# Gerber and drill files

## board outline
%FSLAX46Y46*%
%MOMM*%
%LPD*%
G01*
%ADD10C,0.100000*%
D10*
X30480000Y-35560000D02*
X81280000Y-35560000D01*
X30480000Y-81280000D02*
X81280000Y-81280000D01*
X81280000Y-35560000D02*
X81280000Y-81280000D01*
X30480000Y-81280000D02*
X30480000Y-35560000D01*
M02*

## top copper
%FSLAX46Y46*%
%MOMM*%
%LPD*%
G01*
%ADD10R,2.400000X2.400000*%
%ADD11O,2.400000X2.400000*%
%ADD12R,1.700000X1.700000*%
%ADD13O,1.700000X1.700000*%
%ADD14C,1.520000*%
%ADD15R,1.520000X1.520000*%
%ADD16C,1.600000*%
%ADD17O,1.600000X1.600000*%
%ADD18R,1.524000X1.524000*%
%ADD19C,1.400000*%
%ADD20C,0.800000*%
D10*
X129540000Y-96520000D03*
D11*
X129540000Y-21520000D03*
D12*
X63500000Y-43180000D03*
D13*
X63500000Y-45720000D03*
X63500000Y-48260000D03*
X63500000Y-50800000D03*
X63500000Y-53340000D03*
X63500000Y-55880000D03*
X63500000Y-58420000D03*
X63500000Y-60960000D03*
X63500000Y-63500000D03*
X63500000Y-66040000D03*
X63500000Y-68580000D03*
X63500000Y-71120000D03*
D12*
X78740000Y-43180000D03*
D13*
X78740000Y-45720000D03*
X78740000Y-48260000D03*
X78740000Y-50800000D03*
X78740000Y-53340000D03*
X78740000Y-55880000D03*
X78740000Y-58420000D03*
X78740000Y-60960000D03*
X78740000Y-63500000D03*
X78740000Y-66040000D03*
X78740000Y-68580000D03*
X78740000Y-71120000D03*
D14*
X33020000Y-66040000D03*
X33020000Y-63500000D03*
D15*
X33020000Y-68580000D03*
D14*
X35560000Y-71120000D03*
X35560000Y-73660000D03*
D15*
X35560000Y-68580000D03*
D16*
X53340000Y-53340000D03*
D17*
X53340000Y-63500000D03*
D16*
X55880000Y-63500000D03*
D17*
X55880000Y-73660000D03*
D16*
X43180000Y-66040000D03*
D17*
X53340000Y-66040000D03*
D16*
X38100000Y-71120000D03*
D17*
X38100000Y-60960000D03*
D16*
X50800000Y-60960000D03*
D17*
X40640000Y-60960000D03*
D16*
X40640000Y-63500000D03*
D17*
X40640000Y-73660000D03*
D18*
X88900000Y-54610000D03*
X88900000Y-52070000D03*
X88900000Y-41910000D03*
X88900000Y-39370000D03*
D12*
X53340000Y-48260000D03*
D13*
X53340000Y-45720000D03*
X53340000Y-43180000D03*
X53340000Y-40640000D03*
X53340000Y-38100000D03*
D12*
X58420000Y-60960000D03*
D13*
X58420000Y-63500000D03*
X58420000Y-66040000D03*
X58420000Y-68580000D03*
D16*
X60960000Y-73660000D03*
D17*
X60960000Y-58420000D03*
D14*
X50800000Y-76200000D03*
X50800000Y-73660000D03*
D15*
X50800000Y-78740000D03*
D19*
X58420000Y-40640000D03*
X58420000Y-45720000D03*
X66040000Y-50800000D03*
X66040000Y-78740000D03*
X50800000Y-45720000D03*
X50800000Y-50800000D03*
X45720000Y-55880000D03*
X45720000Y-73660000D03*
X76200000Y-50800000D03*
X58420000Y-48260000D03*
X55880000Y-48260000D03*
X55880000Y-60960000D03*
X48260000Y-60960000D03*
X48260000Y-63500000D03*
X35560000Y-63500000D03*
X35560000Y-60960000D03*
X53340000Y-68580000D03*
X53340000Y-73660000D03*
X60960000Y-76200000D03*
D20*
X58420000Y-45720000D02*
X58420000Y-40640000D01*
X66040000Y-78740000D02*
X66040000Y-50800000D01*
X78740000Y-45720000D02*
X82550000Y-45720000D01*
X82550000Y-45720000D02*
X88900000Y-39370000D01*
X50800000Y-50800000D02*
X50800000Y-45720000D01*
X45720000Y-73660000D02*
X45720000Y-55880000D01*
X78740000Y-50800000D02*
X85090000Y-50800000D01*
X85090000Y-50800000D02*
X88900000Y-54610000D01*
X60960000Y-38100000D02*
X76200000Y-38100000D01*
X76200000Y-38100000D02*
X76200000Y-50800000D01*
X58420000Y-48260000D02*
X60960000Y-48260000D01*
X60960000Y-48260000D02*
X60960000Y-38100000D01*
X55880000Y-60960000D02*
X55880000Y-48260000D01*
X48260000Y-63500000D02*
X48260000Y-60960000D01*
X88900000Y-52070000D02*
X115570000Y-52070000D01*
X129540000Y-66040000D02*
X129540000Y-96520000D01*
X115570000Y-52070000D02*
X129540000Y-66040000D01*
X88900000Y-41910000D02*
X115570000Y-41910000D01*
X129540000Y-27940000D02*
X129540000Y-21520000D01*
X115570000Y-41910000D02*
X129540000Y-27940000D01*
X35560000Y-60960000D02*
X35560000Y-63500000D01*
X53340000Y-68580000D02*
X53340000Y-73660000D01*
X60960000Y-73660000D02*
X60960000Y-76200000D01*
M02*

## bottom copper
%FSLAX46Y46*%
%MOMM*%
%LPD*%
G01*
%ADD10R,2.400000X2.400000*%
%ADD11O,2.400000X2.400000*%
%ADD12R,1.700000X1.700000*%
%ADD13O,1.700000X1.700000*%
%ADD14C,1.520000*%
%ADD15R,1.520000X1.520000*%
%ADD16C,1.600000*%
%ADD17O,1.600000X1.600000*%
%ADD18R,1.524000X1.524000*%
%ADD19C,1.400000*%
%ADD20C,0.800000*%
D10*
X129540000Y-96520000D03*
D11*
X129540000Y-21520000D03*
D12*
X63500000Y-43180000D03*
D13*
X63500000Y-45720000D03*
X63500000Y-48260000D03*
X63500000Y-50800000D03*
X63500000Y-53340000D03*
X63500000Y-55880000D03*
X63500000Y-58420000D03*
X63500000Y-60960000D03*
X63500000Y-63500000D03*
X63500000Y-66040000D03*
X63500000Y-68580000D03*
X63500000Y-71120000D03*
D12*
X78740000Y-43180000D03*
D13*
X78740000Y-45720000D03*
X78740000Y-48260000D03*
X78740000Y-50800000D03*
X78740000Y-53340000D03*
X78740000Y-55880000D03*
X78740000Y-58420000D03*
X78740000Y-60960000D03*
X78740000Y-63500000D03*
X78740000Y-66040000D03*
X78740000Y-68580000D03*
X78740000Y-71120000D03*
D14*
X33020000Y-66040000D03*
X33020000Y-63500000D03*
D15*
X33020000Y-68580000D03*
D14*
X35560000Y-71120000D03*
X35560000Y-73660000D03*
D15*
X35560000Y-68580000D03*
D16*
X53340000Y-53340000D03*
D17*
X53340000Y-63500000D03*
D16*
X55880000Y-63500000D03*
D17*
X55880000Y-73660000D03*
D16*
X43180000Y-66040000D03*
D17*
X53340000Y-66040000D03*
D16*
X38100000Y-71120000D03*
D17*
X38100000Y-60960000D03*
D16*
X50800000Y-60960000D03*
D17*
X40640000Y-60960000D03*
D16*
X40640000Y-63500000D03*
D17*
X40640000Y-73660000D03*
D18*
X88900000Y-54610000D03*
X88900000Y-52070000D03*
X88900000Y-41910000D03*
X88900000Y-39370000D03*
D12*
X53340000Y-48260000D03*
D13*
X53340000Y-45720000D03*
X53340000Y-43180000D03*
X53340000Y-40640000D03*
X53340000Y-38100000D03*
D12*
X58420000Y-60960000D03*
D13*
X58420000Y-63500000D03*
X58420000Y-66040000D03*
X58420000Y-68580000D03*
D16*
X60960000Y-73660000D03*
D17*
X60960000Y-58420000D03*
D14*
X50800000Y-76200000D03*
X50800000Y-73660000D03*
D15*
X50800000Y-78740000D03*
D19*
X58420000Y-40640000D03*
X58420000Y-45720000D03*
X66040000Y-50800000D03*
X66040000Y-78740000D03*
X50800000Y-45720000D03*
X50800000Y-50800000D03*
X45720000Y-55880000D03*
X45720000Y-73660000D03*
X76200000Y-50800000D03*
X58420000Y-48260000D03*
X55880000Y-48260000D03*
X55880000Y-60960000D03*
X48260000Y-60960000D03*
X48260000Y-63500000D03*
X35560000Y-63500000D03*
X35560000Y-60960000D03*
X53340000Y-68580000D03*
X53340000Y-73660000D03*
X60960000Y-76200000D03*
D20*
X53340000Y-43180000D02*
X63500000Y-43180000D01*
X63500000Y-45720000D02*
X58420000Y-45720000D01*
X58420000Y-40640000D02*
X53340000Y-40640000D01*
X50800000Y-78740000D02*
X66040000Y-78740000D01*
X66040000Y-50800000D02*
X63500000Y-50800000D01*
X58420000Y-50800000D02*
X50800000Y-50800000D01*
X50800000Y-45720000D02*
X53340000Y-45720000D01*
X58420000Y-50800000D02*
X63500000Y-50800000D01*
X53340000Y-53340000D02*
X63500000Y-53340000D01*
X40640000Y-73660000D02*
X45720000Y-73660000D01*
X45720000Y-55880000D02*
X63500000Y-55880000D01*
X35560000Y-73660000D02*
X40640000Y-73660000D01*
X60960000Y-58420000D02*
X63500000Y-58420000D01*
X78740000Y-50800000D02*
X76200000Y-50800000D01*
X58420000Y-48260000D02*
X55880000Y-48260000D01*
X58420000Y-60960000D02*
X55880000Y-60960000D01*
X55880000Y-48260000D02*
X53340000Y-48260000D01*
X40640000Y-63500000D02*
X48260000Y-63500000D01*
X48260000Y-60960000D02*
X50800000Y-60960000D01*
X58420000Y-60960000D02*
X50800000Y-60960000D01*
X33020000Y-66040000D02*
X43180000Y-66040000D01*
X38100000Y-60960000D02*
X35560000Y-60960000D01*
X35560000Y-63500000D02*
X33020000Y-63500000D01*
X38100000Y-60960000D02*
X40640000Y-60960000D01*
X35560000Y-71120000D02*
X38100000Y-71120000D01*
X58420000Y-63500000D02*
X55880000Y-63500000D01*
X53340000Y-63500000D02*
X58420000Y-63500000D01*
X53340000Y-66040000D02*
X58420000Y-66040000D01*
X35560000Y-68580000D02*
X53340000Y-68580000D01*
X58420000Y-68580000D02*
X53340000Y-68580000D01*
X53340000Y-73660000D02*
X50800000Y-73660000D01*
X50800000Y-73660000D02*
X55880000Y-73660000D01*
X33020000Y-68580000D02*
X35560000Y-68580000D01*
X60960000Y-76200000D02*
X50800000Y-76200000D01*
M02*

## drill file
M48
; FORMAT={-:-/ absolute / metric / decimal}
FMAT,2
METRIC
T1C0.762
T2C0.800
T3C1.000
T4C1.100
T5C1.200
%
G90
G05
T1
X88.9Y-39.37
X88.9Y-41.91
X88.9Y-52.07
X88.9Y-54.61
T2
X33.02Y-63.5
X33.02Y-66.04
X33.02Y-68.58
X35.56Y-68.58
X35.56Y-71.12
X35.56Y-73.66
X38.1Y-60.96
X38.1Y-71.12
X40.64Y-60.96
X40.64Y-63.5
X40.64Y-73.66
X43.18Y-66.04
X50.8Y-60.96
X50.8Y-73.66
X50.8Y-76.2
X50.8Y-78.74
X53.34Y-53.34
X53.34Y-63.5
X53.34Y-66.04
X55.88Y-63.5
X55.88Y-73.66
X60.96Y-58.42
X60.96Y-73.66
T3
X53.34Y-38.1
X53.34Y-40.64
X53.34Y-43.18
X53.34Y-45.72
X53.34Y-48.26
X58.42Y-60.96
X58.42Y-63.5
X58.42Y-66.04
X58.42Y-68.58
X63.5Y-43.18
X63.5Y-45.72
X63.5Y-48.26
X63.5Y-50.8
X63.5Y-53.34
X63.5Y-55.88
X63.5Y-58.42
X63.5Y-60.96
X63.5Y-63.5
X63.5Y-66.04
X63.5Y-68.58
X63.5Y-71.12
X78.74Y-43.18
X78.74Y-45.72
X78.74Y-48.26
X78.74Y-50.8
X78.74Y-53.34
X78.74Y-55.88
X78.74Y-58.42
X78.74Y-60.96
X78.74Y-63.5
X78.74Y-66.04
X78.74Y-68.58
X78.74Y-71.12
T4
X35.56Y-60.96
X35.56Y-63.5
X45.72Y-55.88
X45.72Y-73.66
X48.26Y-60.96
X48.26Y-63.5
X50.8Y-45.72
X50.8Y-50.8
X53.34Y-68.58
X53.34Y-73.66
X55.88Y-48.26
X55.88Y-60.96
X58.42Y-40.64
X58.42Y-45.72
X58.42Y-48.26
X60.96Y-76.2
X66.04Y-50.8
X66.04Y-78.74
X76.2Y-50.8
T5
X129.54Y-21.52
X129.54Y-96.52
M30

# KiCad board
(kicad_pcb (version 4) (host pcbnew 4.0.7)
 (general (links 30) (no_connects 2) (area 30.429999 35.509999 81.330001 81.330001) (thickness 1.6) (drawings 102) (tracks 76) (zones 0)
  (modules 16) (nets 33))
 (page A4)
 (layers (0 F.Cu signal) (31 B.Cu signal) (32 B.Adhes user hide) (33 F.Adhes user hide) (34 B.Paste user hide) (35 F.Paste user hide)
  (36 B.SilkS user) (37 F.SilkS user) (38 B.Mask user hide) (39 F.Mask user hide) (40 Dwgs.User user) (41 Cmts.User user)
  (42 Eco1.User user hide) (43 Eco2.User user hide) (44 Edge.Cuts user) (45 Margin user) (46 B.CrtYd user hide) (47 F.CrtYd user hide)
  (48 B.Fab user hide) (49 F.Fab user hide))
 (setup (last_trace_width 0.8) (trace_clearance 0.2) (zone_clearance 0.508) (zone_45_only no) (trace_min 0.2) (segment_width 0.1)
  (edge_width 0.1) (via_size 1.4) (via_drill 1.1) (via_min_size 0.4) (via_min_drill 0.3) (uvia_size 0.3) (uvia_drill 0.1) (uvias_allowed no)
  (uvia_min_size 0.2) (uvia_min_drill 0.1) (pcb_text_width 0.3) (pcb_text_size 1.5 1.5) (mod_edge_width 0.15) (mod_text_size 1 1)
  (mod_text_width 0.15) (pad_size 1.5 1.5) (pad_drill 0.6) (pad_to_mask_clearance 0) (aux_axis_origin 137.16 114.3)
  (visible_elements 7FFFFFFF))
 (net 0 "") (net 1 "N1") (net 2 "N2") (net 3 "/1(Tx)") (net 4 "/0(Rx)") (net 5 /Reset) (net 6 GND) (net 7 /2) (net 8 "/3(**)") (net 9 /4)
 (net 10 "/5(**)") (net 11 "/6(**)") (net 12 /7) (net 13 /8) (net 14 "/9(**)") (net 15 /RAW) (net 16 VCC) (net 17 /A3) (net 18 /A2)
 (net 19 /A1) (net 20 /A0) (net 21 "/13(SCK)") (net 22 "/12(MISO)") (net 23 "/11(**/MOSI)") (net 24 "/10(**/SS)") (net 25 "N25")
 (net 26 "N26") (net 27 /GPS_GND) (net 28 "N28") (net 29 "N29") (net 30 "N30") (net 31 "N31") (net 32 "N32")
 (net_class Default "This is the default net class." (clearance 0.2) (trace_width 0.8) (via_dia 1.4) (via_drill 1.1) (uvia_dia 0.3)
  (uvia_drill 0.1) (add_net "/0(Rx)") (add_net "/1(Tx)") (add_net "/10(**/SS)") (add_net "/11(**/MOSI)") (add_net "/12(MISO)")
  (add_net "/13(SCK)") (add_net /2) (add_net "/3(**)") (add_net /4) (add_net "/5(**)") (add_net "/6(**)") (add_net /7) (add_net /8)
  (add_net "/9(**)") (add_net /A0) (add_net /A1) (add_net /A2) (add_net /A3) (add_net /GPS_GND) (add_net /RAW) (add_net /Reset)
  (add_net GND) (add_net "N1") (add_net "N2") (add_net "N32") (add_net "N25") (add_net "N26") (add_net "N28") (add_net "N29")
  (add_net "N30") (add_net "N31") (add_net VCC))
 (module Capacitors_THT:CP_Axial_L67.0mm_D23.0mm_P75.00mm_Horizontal (layer F.Cu) (at 129.54 96.52 90)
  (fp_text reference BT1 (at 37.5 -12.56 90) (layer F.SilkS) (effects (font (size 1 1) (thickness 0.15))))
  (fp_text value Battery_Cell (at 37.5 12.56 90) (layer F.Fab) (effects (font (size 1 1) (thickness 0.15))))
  (pad 1 thru_hole rect (at 0 0 90) (size 2.4 2.4) (drill 1.2) (layers *.Cu *.Mask) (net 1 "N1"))
  (pad 2 thru_hole oval (at 75 0 90) (size 2.4 2.4) (drill 1.2) (layers *.Cu *.Mask) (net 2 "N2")))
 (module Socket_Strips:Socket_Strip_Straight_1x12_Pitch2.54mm (layer F.Cu) (at 63.5 43.18)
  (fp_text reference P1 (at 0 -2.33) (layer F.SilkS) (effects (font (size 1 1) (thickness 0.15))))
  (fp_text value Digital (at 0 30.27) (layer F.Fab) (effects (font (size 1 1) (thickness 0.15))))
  (pad 1 thru_hole rect (at 0 0) (size 1.7 1.7) (drill 1) (layers *.Cu *.Mask) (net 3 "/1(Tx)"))
  (pad 2 thru_hole oval (at 0 2.54) (size 1.7 1.7) (drill 1) (layers *.Cu *.Mask) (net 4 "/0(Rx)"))
  (pad 3 thru_hole oval (at 0 5.08) (size 1.7 1.7) (drill 1) (layers *.Cu *.Mask) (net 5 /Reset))
  (pad 4 thru_hole oval (at 0 7.62) (size 1.7 1.7) (drill 1) (layers *.Cu *.Mask) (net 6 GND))
  (pad 5 thru_hole oval (at 0 10.16) (size 1.7 1.7) (drill 1) (layers *.Cu *.Mask) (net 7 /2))
  (pad 6 thru_hole oval (at 0 12.7) (size 1.7 1.7) (drill 1) (layers *.Cu *.Mask) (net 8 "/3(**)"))
  (pad 7 thru_hole oval (at 0 15.24) (size 1.7 1.7) (drill 1) (layers *.Cu *.Mask) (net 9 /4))
  (pad 8 thru_hole oval (at 0 17.78) (size 1.7 1.7) (drill 1) (layers *.Cu *.Mask) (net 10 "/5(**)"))
  (pad 9 thru_hole oval (at 0 20.32) (size 1.7 1.7) (drill 1) (layers *.Cu *.Mask) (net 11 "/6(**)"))
  (pad 10 thru_hole oval (at 0 22.86) (size 1.7 1.7) (drill 1) (layers *.Cu *.Mask) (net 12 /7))
  (pad 11 thru_hole oval (at 0 25.4) (size 1.7 1.7) (drill 1) (layers *.Cu *.Mask) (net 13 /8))
  (pad 12 thru_hole oval (at 0 27.94) (size 1.7 1.7) (drill 1) (layers *.Cu *.Mask) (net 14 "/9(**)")))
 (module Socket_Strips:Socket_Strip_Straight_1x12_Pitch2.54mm (layer F.Cu) (at 78.74 43.18)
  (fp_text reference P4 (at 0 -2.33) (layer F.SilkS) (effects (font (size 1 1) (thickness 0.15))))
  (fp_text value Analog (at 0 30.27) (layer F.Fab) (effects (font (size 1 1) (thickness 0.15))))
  (pad 1 thru_hole rect (at 0 0) (size 1.7 1.7) (drill 1) (layers *.Cu *.Mask) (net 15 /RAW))
  (pad 2 thru_hole oval (at 0 2.54) (size 1.7 1.7) (drill 1) (layers *.Cu *.Mask) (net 6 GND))
  (pad 3 thru_hole oval (at 0 5.08) (size 1.7 1.7) (drill 1) (layers *.Cu *.Mask) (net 5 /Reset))
  (pad 4 thru_hole oval (at 0 7.62) (size 1.7 1.7) (drill 1) (layers *.Cu *.Mask) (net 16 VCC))
  (pad 5 thru_hole oval (at 0 10.16) (size 1.7 1.7) (drill 1) (layers *.Cu *.Mask) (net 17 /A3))
  (pad 6 thru_hole oval (at 0 12.7) (size 1.7 1.7) (drill 1) (layers *.Cu *.Mask) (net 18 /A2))
  (pad 7 thru_hole oval (at 0 15.24) (size 1.7 1.7) (drill 1) (layers *.Cu *.Mask) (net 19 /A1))
  (pad 8 thru_hole oval (at 0 17.78) (size 1.7 1.7) (drill 1) (layers *.Cu *.Mask) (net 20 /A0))
  (pad 9 thru_hole oval (at 0 20.32) (size 1.7 1.7) (drill 1) (layers *.Cu *.Mask) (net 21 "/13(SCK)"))
  (pad 10 thru_hole oval (at 0 22.86) (size 1.7 1.7) (drill 1) (layers *.Cu *.Mask) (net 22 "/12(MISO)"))
  (pad 11 thru_hole oval (at 0 25.4) (size 1.7 1.7) (drill 1) (layers *.Cu *.Mask) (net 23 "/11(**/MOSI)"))
  (pad 12 thru_hole oval (at 0 27.94) (size 1.7 1.7) (drill 1) (layers *.Cu *.Mask) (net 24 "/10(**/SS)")))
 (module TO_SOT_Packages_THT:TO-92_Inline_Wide (layer F.Cu) (at 33.02 68.58 90)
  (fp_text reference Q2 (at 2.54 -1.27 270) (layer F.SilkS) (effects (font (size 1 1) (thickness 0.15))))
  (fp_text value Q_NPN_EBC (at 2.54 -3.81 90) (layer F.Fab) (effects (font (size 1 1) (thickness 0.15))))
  (pad 2 thru_hole circle (at 2.54 0 180) (size 1.52 1.52) (drill 0.8) (layers *.Cu *.Mask) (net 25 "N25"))
  (pad 3 thru_hole circle (at 5.08 0 180) (size 1.52 1.52) (drill 0.8) (layers *.Cu *.Mask) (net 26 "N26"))
  (pad 1 thru_hole rect (at 0 0 180) (size 1.52 1.52) (drill 0.8) (layers *.Cu *.Mask) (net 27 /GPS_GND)))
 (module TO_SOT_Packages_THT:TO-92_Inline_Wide (layer F.Cu) (at 35.56 68.58 270)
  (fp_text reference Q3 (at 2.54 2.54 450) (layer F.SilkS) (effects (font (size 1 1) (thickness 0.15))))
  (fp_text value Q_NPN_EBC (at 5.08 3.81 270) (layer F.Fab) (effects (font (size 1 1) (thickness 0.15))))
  (pad 2 thru_hole circle (at 2.54 0) (size 1.52 1.52) (drill 0.8) (layers *.Cu *.Mask) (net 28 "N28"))
  (pad 3 thru_hole circle (at 5.08 0) (size 1.52 1.52) (drill 0.8) (layers *.Cu *.Mask) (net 8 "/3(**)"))
  (pad 1 thru_hole rect (at 0 0) (size 1.52 1.52) (drill 0.8) (layers *.Cu *.Mask) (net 27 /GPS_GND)))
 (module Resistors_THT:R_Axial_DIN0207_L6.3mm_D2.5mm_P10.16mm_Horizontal (layer F.Cu) (at 53.34 53.34 270)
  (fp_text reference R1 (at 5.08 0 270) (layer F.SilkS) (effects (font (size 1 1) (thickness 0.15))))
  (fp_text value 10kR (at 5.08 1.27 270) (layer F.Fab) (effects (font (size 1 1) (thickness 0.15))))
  (pad 1 thru_hole circle (at 0 0 270) (size 1.6 1.6) (drill 0.8) (layers *.Cu *.Mask) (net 7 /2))
  (pad 2 thru_hole oval (at 10.16 0 270) (size 1.6 1.6) (drill 0.8) (layers *.Cu *.Mask) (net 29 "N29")))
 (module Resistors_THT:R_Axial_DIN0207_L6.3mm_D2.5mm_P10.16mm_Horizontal (layer F.Cu) (at 55.88 63.5 270)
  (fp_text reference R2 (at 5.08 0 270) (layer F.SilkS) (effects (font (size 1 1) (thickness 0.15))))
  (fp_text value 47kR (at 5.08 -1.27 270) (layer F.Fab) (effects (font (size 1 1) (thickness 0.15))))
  (pad 1 thru_hole circle (at 0 0 270) (size 1.6 1.6) (drill 0.8) (layers *.Cu *.Mask) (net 29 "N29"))
  (pad 2 thru_hole oval (at 10.16 0 270) (size 1.6 1.6) (drill 0.8) (layers *.Cu *.Mask) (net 27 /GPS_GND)))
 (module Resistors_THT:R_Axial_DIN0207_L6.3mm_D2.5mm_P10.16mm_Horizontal (layer F.Cu) (at 43.18 66.04)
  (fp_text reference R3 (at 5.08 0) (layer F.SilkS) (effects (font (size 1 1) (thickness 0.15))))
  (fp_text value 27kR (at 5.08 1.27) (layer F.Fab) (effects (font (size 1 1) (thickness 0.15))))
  (pad 1 thru_hole circle (at 0 0) (size 1.6 1.6) (drill 0.8) (layers *.Cu *.Mask) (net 25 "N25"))
  (pad 2 thru_hole oval (at 10.16 0) (size 1.6 1.6) (drill 0.8) (layers *.Cu *.Mask) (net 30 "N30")))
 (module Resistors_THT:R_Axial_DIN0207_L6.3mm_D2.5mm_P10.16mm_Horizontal (layer F.Cu) (at 38.1 71.12 90)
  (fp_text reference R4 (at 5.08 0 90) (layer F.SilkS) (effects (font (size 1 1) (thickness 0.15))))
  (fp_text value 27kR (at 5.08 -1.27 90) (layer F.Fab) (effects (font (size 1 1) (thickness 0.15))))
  (pad 1 thru_hole circle (at 0 0 90) (size 1.6 1.6) (drill 0.8) (layers *.Cu *.Mask) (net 28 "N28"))
  (pad 2 thru_hole oval (at 10.16 0 90) (size 1.6 1.6) (drill 0.8) (layers *.Cu *.Mask) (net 26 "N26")))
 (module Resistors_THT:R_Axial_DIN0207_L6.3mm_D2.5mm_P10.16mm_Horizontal (layer F.Cu) (at 50.8 60.96 180)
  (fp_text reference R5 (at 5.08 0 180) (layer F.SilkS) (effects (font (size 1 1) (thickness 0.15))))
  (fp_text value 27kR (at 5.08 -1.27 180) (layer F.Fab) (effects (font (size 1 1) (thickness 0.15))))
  (pad 1 thru_hole circle (at 0 0 180) (size 1.6 1.6) (drill 0.8) (layers *.Cu *.Mask) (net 16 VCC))
  (pad 2 thru_hole oval (at 10.16 0 180) (size 1.6 1.6) (drill 0.8) (layers *.Cu *.Mask) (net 26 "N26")))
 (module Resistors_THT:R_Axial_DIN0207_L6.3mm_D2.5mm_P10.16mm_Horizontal (layer F.Cu) (at 40.64 63.5 270)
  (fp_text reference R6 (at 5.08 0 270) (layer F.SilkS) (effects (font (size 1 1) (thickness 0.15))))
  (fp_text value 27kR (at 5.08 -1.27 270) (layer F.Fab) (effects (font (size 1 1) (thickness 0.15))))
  (pad 1 thru_hole circle (at 0 0 270) (size 1.6 1.6) (drill 0.8) (layers *.Cu *.Mask) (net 16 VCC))
  (pad 2 thru_hole oval (at 10.16 0 270) (size 1.6 1.6) (drill 0.8) (layers *.Cu *.Mask) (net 8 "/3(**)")))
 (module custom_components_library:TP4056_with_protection (layer F.Cu) (at 114.3 55.88 180)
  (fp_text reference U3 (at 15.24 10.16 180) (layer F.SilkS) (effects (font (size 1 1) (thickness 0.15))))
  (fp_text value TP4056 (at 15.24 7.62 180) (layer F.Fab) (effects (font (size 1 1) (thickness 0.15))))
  (pad 1 thru_hole rect (at 25.4 1.27 180) (size 1.524 1.524) (drill 0.762) (layers *.Cu *.Mask) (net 16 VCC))
  (pad 2 thru_hole rect (at 25.4 3.81 180) (size 1.524 1.524) (drill 0.762) (layers *.Cu *.Mask) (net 1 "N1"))
  (pad 3 thru_hole rect (at 25.4 13.97 180) (size 1.524 1.524) (drill 0.762) (layers *.Cu *.Mask) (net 2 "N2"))
  (pad 4 thru_hole rect (at 25.4 16.51 180) (size 1.524 1.524) (drill 0.762) (layers *.Cu *.Mask) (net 6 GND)))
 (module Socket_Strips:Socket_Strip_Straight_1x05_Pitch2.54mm (layer F.Cu) (at 53.34 48.26 180)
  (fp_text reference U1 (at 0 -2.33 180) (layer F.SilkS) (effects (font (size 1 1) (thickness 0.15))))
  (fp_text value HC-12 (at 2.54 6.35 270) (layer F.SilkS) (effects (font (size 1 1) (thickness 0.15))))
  (pad 1 thru_hole rect (at 0 0 180) (size 1.7 1.7) (drill 1) (layers *.Cu *.Mask) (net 16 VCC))
  (pad 2 thru_hole oval (at 0 2.54 180) (size 1.7 1.7) (drill 1) (layers *.Cu *.Mask) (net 6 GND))
  (pad 3 thru_hole oval (at 0 5.08 180) (size 1.7 1.7) (drill 1) (layers *.Cu *.Mask) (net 3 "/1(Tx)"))
  (pad 4 thru_hole oval (at 0 7.62 180) (size 1.7 1.7) (drill 1) (layers *.Cu *.Mask) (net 4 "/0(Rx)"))
  (pad 5 thru_hole oval (at 0 10.16 180) (size 1.7 1.7) (drill 1) (layers *.Cu *.Mask) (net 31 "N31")))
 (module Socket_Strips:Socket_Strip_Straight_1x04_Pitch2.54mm (layer F.Cu) (at 58.42 60.96)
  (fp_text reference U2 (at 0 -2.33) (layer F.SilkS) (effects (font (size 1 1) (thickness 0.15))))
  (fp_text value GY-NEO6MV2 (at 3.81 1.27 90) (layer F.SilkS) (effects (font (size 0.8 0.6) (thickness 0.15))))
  (pad 1 thru_hole rect (at 0 0) (size 1.7 1.7) (drill 1) (layers *.Cu *.Mask) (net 16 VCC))
  (pad 2 thru_hole oval (at 0 2.54) (size 1.7 1.7) (drill 1) (layers *.Cu *.Mask) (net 29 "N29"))
  (pad 3 thru_hole oval (at 0 5.08) (size 1.7 1.7) (drill 1) (layers *.Cu *.Mask) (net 30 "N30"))
  (pad 4 thru_hole oval (at 0 7.62) (size 1.7 1.7) (drill 1) (layers *.Cu *.Mask) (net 27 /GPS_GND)))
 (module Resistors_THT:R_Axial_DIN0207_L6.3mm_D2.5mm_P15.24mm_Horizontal (layer F.Cu) (at 60.96 73.66 90)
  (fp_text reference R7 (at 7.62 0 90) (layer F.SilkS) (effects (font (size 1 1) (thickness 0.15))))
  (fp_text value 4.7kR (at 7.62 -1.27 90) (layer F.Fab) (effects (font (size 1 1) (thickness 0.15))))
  (pad 1 thru_hole circle (at 0 0 90) (size 1.6 1.6) (drill 0.8) (layers *.Cu *.Mask) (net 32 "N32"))
  (pad 2 thru_hole oval (at 15.24 0 90) (size 1.6 1.6) (drill 0.8) (layers *.Cu *.Mask) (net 9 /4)))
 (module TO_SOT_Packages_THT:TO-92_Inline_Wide (layer F.Cu) (at 50.8 78.74 90)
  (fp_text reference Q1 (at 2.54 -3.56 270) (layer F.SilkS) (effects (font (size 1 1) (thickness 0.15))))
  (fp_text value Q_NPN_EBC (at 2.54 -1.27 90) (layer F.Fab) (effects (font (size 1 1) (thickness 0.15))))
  (pad 2 thru_hole circle (at 2.54 0 180) (size 1.52 1.52) (drill 0.8) (layers *.Cu *.Mask) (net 32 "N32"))
  (pad 3 thru_hole circle (at 5.08 0 180) (size 1.52 1.52) (drill 0.8) (layers *.Cu *.Mask) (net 27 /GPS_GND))
  (pad 1 thru_hole rect (at 0 0 180) (size 1.52 1.52) (drill 0.8) (layers *.Cu *.Mask) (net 6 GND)))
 (gr_line (start 30.48 35.56) (end 81.28 35.56) (angle 90) (layer Edge.Cuts) (width 0.1))
 (gr_line (start 30.48 81.28) (end 81.28 81.28) (angle 90) (layer Edge.Cuts) (width 0.1))
 (gr_line (start 81.28 35.56) (end 81.28 81.28) (angle 90) (layer Edge.Cuts) (width 0.1))
 (gr_line (start 30.48 81.28) (end 30.48 35.56) (angle 90) (layer Edge.Cuts) (width 0.1))
 (segment (start 53.34 43.18) (end 63.5 43.18) (width 0.8) (layer B.Cu) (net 3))
 (segment (start 63.5 45.72) (end 58.42 45.72) (width 0.8) (layer B.Cu) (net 4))
 (segment (start 58.42 40.64) (end 53.34 40.64) (width 0.8) (layer B.Cu) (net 4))
 (via (at 58.42 40.64) (size 1.4) (drill 1.1) (layers F.Cu B.Cu) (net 4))
 (segment (start 58.42 45.72) (end 58.42 40.64) (width 0.8) (layer F.Cu) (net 4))
 (via (at 58.42 45.72) (size 1.4) (drill 1.1) (layers F.Cu B.Cu) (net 4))
 (segment (start 50.8 78.74) (end 66.04 78.74) (width 0.8) (layer B.Cu) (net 6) (status 10))
 (segment (start 66.04 50.8) (end 63.5 50.8) (width 0.8) (layer B.Cu) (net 6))
 (via (at 66.04 50.8) (size 1.4) (drill 1.1) (layers F.Cu B.Cu) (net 6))
 (segment (start 66.04 78.74) (end 66.04 50.8) (width 0.8) (layer F.Cu) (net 6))
 (via (at 66.04 78.74) (size 1.4) (drill 1.1) (layers F.Cu B.Cu) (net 6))
 (segment (start 78.74 45.72) (end 82.55 45.72) (width 0.8) (layer F.Cu) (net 6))
 (segment (start 82.55 45.72) (end 88.9 39.37) (width 0.8) (layer F.Cu) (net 6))
 (segment (start 58.42 50.8) (end 50.8 50.8) (width 0.8) (layer B.Cu) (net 6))
 (segment (start 50.8 45.72) (end 53.34 45.72) (width 0.8) (layer B.Cu) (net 6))
 (via (at 50.8 45.72) (size 1.4) (drill 1.1) (layers F.Cu B.Cu) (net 6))
 (segment (start 50.8 50.8) (end 50.8 45.72) (width 0.8) (layer F.Cu) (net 6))
 (via (at 50.8 50.8) (size 1.4) (drill 1.1) (layers F.Cu B.Cu) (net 6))
 (segment (start 58.42 50.8) (end 63.5 50.8) (width 0.8) (layer B.Cu) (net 6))
 (segment (start 53.34 53.34) (end 63.5 53.34) (width 0.8) (layer B.Cu) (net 7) (status 10))
 (segment (start 40.64 73.66) (end 45.72 73.66) (width 0.8) (layer B.Cu) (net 8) (status 10))
 (segment (start 45.72 55.88) (end 63.5 55.88) (width 0.8) (layer B.Cu) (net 8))
 (via (at 45.72 55.88) (size 1.4) (drill 1.1) (layers F.Cu B.Cu) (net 8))
 (segment (start 45.72 73.66) (end 45.72 55.88) (width 0.8) (layer F.Cu) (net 8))
 (via (at 45.72 73.66) (size 1.4) (drill 1.1) (layers F.Cu B.Cu) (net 8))
 (segment (start 35.56 73.66) (end 40.64 73.66) (width 0.8) (layer B.Cu) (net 8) (status 10))
 (segment (start 60.96 58.42) (end 63.5 58.42) (width 0.8) (layer B.Cu) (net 9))
 (segment (start 78.74 50.8) (end 85.09 50.8) (width 0.8) (layer F.Cu) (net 16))
 (segment (start 85.09 50.8) (end 88.9 54.61) (width 0.8) (layer F.Cu) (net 16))
 (segment (start 60.96 38.1) (end 76.2 38.1) (width 0.8) (layer F.Cu) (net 16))
 (segment (start 76.2 38.1) (end 76.2 50.8) (width 0.8) (layer F.Cu) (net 16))
 (via (at 76.2 50.8) (size 1.4) (drill 1.1) (layers F.Cu B.Cu) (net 16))
 (segment (start 78.74 50.8) (end 76.2 50.8) (width 0.8) (layer B.Cu) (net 16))
 (via (at 58.42 48.26) (size 1.4) (drill 1.1) (layers F.Cu B.Cu) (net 16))
 (segment (start 58.42 48.26) (end 60.96 48.26) (width 0.8) (layer F.Cu) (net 16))
 (segment (start 60.96 48.26) (end 60.96 38.1) (width 0.8) (layer F.Cu) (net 16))
 (segment (start 58.42 48.26) (end 55.88 48.26) (width 0.8) (layer B.Cu) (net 16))
 (segment (start 58.42 60.96) (end 55.88 60.96) (width 0.8) (layer B.Cu) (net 16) (status 10))
 (segment (start 55.88 48.26) (end 53.34 48.26) (width 0.8) (layer B.Cu) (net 16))
 (via (at 55.88 48.26) (size 1.4) (drill 1.1) (layers F.Cu B.Cu) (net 16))
 (segment (start 55.88 60.96) (end 55.88 48.26) (width 0.8) (layer F.Cu) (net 16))
 (via (at 55.88 60.96) (size 1.4) (drill 1.1) (layers F.Cu B.Cu) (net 16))
 (segment (start 40.64 63.5) (end 48.26 63.5) (width 0.8) (layer B.Cu) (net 16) (status 10))
 (segment (start 48.26 60.96) (end 50.8 60.96) (width 0.8) (layer B.Cu) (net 16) (status 20))
 (via (at 48.26 60.96) (size 1.4) (drill 1.1) (layers F.Cu B.Cu) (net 16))
 (segment (start 48.26 63.5) (end 48.26 60.96) (width 0.8) (layer F.Cu) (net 16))
 (via (at 48.26 63.5) (size 1.4) (drill 1.1) (layers F.Cu B.Cu) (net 16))
 (segment (start 58.42 60.96) (end 50.8 60.96) (width 0.8) (layer B.Cu) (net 16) (status 20))
 (segment (start 88.9 52.07) (end 115.57 52.07) (width 0.8) (layer F.Cu) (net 1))
 (segment (start 129.54 66.04) (end 129.54 96.52) (width 0.8) (layer F.Cu) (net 1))
 (segment (start 115.57 52.07) (end 129.54 66.04) (width 0.8) (layer F.Cu) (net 1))
 (segment (start 88.9 41.91) (end 115.57 41.91) (width 0.8) (layer F.Cu) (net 2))
 (segment (start 129.54 27.94) (end 129.54 21.52) (width 0.8) (layer F.Cu) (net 2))
 (segment (start 115.57 41.91) (end 129.54 27.94) (width 0.8) (layer F.Cu) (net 2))
 (segment (start 33.02 66.04) (end 43.18 66.04) (width 0.8) (layer B.Cu) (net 25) (status 10))
 (segment (start 38.1 60.96) (end 35.56 60.96) (width 0.8) (layer B.Cu) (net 26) (status 10))
 (segment (start 35.56 63.5) (end 33.02 63.5) (width 0.8) (layer B.Cu) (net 26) (status 20))
 (via (at 35.56 63.5) (size 1.4) (drill 1.1) (layers F.Cu B.Cu) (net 26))
 (segment (start 35.56 60.96) (end 35.56 63.5) (width 0.8) (layer F.Cu) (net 26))
 (via (at 35.56 60.96) (size 1.4) (drill 1.1) (layers F.Cu B.Cu) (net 26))
 (segment (start 38.1 60.96) (end 40.64 60.96) (width 0.8) (layer B.Cu) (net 26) (status 10))
 (segment (start 35.56 71.12) (end 38.1 71.12) (width 0.8) (layer B.Cu) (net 28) (status 10))
 (segment (start 58.42 63.5) (end 55.88 63.5) (width 0.8) (layer B.Cu) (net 29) (status 20))
 (segment (start 53.34 63.5) (end 58.42 63.5) (width 0.8) (layer B.Cu) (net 29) (status 10))
 (segment (start 53.34 66.04) (end 58.42 66.04) (width 0.8) (layer B.Cu) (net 30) (status 10))
 (segment (start 35.56 68.58) (end 53.34 68.58) (width 0.8) (layer B.Cu) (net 27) (status 10))
 (segment (start 58.42 68.58) (end 53.34 68.58) (width 0.8) (layer B.Cu) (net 27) (status 10))
 (segment (start 53.34 73.66) (end 50.8 73.66) (width 0.8) (layer B.Cu) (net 27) (status 20))
 (via (at 53.34 68.58) (size 1.4) (drill 1.1) (layers F.Cu B.Cu) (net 27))
 (segment (start 53.34 68.58) (end 53.34 73.66) (width 0.8) (layer F.Cu) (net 27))
 (via (at 53.34 73.66) (size 1.4) (drill 1.1) (layers F.Cu B.Cu) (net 27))
 (segment (start 50.8 73.66) (end 55.88 73.66) (width 0.8) (layer B.Cu) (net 27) (status 10))
 (segment (start 33.02 68.58) (end 35.56 68.58) (width 0.8) (layer B.Cu) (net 27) (status 10))
 (segment (start 60.96 73.66) (end 60.96 76.2) (width 0.8) (layer F.Cu) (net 32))
 (via (at 60.96 76.2) (size 1.4) (drill 1.1) (layers F.Cu B.Cu) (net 32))
 (segment (start 60.96 76.2) (end 50.8 76.2) (width 0.8) (layer B.Cu) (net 32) (status 20)))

